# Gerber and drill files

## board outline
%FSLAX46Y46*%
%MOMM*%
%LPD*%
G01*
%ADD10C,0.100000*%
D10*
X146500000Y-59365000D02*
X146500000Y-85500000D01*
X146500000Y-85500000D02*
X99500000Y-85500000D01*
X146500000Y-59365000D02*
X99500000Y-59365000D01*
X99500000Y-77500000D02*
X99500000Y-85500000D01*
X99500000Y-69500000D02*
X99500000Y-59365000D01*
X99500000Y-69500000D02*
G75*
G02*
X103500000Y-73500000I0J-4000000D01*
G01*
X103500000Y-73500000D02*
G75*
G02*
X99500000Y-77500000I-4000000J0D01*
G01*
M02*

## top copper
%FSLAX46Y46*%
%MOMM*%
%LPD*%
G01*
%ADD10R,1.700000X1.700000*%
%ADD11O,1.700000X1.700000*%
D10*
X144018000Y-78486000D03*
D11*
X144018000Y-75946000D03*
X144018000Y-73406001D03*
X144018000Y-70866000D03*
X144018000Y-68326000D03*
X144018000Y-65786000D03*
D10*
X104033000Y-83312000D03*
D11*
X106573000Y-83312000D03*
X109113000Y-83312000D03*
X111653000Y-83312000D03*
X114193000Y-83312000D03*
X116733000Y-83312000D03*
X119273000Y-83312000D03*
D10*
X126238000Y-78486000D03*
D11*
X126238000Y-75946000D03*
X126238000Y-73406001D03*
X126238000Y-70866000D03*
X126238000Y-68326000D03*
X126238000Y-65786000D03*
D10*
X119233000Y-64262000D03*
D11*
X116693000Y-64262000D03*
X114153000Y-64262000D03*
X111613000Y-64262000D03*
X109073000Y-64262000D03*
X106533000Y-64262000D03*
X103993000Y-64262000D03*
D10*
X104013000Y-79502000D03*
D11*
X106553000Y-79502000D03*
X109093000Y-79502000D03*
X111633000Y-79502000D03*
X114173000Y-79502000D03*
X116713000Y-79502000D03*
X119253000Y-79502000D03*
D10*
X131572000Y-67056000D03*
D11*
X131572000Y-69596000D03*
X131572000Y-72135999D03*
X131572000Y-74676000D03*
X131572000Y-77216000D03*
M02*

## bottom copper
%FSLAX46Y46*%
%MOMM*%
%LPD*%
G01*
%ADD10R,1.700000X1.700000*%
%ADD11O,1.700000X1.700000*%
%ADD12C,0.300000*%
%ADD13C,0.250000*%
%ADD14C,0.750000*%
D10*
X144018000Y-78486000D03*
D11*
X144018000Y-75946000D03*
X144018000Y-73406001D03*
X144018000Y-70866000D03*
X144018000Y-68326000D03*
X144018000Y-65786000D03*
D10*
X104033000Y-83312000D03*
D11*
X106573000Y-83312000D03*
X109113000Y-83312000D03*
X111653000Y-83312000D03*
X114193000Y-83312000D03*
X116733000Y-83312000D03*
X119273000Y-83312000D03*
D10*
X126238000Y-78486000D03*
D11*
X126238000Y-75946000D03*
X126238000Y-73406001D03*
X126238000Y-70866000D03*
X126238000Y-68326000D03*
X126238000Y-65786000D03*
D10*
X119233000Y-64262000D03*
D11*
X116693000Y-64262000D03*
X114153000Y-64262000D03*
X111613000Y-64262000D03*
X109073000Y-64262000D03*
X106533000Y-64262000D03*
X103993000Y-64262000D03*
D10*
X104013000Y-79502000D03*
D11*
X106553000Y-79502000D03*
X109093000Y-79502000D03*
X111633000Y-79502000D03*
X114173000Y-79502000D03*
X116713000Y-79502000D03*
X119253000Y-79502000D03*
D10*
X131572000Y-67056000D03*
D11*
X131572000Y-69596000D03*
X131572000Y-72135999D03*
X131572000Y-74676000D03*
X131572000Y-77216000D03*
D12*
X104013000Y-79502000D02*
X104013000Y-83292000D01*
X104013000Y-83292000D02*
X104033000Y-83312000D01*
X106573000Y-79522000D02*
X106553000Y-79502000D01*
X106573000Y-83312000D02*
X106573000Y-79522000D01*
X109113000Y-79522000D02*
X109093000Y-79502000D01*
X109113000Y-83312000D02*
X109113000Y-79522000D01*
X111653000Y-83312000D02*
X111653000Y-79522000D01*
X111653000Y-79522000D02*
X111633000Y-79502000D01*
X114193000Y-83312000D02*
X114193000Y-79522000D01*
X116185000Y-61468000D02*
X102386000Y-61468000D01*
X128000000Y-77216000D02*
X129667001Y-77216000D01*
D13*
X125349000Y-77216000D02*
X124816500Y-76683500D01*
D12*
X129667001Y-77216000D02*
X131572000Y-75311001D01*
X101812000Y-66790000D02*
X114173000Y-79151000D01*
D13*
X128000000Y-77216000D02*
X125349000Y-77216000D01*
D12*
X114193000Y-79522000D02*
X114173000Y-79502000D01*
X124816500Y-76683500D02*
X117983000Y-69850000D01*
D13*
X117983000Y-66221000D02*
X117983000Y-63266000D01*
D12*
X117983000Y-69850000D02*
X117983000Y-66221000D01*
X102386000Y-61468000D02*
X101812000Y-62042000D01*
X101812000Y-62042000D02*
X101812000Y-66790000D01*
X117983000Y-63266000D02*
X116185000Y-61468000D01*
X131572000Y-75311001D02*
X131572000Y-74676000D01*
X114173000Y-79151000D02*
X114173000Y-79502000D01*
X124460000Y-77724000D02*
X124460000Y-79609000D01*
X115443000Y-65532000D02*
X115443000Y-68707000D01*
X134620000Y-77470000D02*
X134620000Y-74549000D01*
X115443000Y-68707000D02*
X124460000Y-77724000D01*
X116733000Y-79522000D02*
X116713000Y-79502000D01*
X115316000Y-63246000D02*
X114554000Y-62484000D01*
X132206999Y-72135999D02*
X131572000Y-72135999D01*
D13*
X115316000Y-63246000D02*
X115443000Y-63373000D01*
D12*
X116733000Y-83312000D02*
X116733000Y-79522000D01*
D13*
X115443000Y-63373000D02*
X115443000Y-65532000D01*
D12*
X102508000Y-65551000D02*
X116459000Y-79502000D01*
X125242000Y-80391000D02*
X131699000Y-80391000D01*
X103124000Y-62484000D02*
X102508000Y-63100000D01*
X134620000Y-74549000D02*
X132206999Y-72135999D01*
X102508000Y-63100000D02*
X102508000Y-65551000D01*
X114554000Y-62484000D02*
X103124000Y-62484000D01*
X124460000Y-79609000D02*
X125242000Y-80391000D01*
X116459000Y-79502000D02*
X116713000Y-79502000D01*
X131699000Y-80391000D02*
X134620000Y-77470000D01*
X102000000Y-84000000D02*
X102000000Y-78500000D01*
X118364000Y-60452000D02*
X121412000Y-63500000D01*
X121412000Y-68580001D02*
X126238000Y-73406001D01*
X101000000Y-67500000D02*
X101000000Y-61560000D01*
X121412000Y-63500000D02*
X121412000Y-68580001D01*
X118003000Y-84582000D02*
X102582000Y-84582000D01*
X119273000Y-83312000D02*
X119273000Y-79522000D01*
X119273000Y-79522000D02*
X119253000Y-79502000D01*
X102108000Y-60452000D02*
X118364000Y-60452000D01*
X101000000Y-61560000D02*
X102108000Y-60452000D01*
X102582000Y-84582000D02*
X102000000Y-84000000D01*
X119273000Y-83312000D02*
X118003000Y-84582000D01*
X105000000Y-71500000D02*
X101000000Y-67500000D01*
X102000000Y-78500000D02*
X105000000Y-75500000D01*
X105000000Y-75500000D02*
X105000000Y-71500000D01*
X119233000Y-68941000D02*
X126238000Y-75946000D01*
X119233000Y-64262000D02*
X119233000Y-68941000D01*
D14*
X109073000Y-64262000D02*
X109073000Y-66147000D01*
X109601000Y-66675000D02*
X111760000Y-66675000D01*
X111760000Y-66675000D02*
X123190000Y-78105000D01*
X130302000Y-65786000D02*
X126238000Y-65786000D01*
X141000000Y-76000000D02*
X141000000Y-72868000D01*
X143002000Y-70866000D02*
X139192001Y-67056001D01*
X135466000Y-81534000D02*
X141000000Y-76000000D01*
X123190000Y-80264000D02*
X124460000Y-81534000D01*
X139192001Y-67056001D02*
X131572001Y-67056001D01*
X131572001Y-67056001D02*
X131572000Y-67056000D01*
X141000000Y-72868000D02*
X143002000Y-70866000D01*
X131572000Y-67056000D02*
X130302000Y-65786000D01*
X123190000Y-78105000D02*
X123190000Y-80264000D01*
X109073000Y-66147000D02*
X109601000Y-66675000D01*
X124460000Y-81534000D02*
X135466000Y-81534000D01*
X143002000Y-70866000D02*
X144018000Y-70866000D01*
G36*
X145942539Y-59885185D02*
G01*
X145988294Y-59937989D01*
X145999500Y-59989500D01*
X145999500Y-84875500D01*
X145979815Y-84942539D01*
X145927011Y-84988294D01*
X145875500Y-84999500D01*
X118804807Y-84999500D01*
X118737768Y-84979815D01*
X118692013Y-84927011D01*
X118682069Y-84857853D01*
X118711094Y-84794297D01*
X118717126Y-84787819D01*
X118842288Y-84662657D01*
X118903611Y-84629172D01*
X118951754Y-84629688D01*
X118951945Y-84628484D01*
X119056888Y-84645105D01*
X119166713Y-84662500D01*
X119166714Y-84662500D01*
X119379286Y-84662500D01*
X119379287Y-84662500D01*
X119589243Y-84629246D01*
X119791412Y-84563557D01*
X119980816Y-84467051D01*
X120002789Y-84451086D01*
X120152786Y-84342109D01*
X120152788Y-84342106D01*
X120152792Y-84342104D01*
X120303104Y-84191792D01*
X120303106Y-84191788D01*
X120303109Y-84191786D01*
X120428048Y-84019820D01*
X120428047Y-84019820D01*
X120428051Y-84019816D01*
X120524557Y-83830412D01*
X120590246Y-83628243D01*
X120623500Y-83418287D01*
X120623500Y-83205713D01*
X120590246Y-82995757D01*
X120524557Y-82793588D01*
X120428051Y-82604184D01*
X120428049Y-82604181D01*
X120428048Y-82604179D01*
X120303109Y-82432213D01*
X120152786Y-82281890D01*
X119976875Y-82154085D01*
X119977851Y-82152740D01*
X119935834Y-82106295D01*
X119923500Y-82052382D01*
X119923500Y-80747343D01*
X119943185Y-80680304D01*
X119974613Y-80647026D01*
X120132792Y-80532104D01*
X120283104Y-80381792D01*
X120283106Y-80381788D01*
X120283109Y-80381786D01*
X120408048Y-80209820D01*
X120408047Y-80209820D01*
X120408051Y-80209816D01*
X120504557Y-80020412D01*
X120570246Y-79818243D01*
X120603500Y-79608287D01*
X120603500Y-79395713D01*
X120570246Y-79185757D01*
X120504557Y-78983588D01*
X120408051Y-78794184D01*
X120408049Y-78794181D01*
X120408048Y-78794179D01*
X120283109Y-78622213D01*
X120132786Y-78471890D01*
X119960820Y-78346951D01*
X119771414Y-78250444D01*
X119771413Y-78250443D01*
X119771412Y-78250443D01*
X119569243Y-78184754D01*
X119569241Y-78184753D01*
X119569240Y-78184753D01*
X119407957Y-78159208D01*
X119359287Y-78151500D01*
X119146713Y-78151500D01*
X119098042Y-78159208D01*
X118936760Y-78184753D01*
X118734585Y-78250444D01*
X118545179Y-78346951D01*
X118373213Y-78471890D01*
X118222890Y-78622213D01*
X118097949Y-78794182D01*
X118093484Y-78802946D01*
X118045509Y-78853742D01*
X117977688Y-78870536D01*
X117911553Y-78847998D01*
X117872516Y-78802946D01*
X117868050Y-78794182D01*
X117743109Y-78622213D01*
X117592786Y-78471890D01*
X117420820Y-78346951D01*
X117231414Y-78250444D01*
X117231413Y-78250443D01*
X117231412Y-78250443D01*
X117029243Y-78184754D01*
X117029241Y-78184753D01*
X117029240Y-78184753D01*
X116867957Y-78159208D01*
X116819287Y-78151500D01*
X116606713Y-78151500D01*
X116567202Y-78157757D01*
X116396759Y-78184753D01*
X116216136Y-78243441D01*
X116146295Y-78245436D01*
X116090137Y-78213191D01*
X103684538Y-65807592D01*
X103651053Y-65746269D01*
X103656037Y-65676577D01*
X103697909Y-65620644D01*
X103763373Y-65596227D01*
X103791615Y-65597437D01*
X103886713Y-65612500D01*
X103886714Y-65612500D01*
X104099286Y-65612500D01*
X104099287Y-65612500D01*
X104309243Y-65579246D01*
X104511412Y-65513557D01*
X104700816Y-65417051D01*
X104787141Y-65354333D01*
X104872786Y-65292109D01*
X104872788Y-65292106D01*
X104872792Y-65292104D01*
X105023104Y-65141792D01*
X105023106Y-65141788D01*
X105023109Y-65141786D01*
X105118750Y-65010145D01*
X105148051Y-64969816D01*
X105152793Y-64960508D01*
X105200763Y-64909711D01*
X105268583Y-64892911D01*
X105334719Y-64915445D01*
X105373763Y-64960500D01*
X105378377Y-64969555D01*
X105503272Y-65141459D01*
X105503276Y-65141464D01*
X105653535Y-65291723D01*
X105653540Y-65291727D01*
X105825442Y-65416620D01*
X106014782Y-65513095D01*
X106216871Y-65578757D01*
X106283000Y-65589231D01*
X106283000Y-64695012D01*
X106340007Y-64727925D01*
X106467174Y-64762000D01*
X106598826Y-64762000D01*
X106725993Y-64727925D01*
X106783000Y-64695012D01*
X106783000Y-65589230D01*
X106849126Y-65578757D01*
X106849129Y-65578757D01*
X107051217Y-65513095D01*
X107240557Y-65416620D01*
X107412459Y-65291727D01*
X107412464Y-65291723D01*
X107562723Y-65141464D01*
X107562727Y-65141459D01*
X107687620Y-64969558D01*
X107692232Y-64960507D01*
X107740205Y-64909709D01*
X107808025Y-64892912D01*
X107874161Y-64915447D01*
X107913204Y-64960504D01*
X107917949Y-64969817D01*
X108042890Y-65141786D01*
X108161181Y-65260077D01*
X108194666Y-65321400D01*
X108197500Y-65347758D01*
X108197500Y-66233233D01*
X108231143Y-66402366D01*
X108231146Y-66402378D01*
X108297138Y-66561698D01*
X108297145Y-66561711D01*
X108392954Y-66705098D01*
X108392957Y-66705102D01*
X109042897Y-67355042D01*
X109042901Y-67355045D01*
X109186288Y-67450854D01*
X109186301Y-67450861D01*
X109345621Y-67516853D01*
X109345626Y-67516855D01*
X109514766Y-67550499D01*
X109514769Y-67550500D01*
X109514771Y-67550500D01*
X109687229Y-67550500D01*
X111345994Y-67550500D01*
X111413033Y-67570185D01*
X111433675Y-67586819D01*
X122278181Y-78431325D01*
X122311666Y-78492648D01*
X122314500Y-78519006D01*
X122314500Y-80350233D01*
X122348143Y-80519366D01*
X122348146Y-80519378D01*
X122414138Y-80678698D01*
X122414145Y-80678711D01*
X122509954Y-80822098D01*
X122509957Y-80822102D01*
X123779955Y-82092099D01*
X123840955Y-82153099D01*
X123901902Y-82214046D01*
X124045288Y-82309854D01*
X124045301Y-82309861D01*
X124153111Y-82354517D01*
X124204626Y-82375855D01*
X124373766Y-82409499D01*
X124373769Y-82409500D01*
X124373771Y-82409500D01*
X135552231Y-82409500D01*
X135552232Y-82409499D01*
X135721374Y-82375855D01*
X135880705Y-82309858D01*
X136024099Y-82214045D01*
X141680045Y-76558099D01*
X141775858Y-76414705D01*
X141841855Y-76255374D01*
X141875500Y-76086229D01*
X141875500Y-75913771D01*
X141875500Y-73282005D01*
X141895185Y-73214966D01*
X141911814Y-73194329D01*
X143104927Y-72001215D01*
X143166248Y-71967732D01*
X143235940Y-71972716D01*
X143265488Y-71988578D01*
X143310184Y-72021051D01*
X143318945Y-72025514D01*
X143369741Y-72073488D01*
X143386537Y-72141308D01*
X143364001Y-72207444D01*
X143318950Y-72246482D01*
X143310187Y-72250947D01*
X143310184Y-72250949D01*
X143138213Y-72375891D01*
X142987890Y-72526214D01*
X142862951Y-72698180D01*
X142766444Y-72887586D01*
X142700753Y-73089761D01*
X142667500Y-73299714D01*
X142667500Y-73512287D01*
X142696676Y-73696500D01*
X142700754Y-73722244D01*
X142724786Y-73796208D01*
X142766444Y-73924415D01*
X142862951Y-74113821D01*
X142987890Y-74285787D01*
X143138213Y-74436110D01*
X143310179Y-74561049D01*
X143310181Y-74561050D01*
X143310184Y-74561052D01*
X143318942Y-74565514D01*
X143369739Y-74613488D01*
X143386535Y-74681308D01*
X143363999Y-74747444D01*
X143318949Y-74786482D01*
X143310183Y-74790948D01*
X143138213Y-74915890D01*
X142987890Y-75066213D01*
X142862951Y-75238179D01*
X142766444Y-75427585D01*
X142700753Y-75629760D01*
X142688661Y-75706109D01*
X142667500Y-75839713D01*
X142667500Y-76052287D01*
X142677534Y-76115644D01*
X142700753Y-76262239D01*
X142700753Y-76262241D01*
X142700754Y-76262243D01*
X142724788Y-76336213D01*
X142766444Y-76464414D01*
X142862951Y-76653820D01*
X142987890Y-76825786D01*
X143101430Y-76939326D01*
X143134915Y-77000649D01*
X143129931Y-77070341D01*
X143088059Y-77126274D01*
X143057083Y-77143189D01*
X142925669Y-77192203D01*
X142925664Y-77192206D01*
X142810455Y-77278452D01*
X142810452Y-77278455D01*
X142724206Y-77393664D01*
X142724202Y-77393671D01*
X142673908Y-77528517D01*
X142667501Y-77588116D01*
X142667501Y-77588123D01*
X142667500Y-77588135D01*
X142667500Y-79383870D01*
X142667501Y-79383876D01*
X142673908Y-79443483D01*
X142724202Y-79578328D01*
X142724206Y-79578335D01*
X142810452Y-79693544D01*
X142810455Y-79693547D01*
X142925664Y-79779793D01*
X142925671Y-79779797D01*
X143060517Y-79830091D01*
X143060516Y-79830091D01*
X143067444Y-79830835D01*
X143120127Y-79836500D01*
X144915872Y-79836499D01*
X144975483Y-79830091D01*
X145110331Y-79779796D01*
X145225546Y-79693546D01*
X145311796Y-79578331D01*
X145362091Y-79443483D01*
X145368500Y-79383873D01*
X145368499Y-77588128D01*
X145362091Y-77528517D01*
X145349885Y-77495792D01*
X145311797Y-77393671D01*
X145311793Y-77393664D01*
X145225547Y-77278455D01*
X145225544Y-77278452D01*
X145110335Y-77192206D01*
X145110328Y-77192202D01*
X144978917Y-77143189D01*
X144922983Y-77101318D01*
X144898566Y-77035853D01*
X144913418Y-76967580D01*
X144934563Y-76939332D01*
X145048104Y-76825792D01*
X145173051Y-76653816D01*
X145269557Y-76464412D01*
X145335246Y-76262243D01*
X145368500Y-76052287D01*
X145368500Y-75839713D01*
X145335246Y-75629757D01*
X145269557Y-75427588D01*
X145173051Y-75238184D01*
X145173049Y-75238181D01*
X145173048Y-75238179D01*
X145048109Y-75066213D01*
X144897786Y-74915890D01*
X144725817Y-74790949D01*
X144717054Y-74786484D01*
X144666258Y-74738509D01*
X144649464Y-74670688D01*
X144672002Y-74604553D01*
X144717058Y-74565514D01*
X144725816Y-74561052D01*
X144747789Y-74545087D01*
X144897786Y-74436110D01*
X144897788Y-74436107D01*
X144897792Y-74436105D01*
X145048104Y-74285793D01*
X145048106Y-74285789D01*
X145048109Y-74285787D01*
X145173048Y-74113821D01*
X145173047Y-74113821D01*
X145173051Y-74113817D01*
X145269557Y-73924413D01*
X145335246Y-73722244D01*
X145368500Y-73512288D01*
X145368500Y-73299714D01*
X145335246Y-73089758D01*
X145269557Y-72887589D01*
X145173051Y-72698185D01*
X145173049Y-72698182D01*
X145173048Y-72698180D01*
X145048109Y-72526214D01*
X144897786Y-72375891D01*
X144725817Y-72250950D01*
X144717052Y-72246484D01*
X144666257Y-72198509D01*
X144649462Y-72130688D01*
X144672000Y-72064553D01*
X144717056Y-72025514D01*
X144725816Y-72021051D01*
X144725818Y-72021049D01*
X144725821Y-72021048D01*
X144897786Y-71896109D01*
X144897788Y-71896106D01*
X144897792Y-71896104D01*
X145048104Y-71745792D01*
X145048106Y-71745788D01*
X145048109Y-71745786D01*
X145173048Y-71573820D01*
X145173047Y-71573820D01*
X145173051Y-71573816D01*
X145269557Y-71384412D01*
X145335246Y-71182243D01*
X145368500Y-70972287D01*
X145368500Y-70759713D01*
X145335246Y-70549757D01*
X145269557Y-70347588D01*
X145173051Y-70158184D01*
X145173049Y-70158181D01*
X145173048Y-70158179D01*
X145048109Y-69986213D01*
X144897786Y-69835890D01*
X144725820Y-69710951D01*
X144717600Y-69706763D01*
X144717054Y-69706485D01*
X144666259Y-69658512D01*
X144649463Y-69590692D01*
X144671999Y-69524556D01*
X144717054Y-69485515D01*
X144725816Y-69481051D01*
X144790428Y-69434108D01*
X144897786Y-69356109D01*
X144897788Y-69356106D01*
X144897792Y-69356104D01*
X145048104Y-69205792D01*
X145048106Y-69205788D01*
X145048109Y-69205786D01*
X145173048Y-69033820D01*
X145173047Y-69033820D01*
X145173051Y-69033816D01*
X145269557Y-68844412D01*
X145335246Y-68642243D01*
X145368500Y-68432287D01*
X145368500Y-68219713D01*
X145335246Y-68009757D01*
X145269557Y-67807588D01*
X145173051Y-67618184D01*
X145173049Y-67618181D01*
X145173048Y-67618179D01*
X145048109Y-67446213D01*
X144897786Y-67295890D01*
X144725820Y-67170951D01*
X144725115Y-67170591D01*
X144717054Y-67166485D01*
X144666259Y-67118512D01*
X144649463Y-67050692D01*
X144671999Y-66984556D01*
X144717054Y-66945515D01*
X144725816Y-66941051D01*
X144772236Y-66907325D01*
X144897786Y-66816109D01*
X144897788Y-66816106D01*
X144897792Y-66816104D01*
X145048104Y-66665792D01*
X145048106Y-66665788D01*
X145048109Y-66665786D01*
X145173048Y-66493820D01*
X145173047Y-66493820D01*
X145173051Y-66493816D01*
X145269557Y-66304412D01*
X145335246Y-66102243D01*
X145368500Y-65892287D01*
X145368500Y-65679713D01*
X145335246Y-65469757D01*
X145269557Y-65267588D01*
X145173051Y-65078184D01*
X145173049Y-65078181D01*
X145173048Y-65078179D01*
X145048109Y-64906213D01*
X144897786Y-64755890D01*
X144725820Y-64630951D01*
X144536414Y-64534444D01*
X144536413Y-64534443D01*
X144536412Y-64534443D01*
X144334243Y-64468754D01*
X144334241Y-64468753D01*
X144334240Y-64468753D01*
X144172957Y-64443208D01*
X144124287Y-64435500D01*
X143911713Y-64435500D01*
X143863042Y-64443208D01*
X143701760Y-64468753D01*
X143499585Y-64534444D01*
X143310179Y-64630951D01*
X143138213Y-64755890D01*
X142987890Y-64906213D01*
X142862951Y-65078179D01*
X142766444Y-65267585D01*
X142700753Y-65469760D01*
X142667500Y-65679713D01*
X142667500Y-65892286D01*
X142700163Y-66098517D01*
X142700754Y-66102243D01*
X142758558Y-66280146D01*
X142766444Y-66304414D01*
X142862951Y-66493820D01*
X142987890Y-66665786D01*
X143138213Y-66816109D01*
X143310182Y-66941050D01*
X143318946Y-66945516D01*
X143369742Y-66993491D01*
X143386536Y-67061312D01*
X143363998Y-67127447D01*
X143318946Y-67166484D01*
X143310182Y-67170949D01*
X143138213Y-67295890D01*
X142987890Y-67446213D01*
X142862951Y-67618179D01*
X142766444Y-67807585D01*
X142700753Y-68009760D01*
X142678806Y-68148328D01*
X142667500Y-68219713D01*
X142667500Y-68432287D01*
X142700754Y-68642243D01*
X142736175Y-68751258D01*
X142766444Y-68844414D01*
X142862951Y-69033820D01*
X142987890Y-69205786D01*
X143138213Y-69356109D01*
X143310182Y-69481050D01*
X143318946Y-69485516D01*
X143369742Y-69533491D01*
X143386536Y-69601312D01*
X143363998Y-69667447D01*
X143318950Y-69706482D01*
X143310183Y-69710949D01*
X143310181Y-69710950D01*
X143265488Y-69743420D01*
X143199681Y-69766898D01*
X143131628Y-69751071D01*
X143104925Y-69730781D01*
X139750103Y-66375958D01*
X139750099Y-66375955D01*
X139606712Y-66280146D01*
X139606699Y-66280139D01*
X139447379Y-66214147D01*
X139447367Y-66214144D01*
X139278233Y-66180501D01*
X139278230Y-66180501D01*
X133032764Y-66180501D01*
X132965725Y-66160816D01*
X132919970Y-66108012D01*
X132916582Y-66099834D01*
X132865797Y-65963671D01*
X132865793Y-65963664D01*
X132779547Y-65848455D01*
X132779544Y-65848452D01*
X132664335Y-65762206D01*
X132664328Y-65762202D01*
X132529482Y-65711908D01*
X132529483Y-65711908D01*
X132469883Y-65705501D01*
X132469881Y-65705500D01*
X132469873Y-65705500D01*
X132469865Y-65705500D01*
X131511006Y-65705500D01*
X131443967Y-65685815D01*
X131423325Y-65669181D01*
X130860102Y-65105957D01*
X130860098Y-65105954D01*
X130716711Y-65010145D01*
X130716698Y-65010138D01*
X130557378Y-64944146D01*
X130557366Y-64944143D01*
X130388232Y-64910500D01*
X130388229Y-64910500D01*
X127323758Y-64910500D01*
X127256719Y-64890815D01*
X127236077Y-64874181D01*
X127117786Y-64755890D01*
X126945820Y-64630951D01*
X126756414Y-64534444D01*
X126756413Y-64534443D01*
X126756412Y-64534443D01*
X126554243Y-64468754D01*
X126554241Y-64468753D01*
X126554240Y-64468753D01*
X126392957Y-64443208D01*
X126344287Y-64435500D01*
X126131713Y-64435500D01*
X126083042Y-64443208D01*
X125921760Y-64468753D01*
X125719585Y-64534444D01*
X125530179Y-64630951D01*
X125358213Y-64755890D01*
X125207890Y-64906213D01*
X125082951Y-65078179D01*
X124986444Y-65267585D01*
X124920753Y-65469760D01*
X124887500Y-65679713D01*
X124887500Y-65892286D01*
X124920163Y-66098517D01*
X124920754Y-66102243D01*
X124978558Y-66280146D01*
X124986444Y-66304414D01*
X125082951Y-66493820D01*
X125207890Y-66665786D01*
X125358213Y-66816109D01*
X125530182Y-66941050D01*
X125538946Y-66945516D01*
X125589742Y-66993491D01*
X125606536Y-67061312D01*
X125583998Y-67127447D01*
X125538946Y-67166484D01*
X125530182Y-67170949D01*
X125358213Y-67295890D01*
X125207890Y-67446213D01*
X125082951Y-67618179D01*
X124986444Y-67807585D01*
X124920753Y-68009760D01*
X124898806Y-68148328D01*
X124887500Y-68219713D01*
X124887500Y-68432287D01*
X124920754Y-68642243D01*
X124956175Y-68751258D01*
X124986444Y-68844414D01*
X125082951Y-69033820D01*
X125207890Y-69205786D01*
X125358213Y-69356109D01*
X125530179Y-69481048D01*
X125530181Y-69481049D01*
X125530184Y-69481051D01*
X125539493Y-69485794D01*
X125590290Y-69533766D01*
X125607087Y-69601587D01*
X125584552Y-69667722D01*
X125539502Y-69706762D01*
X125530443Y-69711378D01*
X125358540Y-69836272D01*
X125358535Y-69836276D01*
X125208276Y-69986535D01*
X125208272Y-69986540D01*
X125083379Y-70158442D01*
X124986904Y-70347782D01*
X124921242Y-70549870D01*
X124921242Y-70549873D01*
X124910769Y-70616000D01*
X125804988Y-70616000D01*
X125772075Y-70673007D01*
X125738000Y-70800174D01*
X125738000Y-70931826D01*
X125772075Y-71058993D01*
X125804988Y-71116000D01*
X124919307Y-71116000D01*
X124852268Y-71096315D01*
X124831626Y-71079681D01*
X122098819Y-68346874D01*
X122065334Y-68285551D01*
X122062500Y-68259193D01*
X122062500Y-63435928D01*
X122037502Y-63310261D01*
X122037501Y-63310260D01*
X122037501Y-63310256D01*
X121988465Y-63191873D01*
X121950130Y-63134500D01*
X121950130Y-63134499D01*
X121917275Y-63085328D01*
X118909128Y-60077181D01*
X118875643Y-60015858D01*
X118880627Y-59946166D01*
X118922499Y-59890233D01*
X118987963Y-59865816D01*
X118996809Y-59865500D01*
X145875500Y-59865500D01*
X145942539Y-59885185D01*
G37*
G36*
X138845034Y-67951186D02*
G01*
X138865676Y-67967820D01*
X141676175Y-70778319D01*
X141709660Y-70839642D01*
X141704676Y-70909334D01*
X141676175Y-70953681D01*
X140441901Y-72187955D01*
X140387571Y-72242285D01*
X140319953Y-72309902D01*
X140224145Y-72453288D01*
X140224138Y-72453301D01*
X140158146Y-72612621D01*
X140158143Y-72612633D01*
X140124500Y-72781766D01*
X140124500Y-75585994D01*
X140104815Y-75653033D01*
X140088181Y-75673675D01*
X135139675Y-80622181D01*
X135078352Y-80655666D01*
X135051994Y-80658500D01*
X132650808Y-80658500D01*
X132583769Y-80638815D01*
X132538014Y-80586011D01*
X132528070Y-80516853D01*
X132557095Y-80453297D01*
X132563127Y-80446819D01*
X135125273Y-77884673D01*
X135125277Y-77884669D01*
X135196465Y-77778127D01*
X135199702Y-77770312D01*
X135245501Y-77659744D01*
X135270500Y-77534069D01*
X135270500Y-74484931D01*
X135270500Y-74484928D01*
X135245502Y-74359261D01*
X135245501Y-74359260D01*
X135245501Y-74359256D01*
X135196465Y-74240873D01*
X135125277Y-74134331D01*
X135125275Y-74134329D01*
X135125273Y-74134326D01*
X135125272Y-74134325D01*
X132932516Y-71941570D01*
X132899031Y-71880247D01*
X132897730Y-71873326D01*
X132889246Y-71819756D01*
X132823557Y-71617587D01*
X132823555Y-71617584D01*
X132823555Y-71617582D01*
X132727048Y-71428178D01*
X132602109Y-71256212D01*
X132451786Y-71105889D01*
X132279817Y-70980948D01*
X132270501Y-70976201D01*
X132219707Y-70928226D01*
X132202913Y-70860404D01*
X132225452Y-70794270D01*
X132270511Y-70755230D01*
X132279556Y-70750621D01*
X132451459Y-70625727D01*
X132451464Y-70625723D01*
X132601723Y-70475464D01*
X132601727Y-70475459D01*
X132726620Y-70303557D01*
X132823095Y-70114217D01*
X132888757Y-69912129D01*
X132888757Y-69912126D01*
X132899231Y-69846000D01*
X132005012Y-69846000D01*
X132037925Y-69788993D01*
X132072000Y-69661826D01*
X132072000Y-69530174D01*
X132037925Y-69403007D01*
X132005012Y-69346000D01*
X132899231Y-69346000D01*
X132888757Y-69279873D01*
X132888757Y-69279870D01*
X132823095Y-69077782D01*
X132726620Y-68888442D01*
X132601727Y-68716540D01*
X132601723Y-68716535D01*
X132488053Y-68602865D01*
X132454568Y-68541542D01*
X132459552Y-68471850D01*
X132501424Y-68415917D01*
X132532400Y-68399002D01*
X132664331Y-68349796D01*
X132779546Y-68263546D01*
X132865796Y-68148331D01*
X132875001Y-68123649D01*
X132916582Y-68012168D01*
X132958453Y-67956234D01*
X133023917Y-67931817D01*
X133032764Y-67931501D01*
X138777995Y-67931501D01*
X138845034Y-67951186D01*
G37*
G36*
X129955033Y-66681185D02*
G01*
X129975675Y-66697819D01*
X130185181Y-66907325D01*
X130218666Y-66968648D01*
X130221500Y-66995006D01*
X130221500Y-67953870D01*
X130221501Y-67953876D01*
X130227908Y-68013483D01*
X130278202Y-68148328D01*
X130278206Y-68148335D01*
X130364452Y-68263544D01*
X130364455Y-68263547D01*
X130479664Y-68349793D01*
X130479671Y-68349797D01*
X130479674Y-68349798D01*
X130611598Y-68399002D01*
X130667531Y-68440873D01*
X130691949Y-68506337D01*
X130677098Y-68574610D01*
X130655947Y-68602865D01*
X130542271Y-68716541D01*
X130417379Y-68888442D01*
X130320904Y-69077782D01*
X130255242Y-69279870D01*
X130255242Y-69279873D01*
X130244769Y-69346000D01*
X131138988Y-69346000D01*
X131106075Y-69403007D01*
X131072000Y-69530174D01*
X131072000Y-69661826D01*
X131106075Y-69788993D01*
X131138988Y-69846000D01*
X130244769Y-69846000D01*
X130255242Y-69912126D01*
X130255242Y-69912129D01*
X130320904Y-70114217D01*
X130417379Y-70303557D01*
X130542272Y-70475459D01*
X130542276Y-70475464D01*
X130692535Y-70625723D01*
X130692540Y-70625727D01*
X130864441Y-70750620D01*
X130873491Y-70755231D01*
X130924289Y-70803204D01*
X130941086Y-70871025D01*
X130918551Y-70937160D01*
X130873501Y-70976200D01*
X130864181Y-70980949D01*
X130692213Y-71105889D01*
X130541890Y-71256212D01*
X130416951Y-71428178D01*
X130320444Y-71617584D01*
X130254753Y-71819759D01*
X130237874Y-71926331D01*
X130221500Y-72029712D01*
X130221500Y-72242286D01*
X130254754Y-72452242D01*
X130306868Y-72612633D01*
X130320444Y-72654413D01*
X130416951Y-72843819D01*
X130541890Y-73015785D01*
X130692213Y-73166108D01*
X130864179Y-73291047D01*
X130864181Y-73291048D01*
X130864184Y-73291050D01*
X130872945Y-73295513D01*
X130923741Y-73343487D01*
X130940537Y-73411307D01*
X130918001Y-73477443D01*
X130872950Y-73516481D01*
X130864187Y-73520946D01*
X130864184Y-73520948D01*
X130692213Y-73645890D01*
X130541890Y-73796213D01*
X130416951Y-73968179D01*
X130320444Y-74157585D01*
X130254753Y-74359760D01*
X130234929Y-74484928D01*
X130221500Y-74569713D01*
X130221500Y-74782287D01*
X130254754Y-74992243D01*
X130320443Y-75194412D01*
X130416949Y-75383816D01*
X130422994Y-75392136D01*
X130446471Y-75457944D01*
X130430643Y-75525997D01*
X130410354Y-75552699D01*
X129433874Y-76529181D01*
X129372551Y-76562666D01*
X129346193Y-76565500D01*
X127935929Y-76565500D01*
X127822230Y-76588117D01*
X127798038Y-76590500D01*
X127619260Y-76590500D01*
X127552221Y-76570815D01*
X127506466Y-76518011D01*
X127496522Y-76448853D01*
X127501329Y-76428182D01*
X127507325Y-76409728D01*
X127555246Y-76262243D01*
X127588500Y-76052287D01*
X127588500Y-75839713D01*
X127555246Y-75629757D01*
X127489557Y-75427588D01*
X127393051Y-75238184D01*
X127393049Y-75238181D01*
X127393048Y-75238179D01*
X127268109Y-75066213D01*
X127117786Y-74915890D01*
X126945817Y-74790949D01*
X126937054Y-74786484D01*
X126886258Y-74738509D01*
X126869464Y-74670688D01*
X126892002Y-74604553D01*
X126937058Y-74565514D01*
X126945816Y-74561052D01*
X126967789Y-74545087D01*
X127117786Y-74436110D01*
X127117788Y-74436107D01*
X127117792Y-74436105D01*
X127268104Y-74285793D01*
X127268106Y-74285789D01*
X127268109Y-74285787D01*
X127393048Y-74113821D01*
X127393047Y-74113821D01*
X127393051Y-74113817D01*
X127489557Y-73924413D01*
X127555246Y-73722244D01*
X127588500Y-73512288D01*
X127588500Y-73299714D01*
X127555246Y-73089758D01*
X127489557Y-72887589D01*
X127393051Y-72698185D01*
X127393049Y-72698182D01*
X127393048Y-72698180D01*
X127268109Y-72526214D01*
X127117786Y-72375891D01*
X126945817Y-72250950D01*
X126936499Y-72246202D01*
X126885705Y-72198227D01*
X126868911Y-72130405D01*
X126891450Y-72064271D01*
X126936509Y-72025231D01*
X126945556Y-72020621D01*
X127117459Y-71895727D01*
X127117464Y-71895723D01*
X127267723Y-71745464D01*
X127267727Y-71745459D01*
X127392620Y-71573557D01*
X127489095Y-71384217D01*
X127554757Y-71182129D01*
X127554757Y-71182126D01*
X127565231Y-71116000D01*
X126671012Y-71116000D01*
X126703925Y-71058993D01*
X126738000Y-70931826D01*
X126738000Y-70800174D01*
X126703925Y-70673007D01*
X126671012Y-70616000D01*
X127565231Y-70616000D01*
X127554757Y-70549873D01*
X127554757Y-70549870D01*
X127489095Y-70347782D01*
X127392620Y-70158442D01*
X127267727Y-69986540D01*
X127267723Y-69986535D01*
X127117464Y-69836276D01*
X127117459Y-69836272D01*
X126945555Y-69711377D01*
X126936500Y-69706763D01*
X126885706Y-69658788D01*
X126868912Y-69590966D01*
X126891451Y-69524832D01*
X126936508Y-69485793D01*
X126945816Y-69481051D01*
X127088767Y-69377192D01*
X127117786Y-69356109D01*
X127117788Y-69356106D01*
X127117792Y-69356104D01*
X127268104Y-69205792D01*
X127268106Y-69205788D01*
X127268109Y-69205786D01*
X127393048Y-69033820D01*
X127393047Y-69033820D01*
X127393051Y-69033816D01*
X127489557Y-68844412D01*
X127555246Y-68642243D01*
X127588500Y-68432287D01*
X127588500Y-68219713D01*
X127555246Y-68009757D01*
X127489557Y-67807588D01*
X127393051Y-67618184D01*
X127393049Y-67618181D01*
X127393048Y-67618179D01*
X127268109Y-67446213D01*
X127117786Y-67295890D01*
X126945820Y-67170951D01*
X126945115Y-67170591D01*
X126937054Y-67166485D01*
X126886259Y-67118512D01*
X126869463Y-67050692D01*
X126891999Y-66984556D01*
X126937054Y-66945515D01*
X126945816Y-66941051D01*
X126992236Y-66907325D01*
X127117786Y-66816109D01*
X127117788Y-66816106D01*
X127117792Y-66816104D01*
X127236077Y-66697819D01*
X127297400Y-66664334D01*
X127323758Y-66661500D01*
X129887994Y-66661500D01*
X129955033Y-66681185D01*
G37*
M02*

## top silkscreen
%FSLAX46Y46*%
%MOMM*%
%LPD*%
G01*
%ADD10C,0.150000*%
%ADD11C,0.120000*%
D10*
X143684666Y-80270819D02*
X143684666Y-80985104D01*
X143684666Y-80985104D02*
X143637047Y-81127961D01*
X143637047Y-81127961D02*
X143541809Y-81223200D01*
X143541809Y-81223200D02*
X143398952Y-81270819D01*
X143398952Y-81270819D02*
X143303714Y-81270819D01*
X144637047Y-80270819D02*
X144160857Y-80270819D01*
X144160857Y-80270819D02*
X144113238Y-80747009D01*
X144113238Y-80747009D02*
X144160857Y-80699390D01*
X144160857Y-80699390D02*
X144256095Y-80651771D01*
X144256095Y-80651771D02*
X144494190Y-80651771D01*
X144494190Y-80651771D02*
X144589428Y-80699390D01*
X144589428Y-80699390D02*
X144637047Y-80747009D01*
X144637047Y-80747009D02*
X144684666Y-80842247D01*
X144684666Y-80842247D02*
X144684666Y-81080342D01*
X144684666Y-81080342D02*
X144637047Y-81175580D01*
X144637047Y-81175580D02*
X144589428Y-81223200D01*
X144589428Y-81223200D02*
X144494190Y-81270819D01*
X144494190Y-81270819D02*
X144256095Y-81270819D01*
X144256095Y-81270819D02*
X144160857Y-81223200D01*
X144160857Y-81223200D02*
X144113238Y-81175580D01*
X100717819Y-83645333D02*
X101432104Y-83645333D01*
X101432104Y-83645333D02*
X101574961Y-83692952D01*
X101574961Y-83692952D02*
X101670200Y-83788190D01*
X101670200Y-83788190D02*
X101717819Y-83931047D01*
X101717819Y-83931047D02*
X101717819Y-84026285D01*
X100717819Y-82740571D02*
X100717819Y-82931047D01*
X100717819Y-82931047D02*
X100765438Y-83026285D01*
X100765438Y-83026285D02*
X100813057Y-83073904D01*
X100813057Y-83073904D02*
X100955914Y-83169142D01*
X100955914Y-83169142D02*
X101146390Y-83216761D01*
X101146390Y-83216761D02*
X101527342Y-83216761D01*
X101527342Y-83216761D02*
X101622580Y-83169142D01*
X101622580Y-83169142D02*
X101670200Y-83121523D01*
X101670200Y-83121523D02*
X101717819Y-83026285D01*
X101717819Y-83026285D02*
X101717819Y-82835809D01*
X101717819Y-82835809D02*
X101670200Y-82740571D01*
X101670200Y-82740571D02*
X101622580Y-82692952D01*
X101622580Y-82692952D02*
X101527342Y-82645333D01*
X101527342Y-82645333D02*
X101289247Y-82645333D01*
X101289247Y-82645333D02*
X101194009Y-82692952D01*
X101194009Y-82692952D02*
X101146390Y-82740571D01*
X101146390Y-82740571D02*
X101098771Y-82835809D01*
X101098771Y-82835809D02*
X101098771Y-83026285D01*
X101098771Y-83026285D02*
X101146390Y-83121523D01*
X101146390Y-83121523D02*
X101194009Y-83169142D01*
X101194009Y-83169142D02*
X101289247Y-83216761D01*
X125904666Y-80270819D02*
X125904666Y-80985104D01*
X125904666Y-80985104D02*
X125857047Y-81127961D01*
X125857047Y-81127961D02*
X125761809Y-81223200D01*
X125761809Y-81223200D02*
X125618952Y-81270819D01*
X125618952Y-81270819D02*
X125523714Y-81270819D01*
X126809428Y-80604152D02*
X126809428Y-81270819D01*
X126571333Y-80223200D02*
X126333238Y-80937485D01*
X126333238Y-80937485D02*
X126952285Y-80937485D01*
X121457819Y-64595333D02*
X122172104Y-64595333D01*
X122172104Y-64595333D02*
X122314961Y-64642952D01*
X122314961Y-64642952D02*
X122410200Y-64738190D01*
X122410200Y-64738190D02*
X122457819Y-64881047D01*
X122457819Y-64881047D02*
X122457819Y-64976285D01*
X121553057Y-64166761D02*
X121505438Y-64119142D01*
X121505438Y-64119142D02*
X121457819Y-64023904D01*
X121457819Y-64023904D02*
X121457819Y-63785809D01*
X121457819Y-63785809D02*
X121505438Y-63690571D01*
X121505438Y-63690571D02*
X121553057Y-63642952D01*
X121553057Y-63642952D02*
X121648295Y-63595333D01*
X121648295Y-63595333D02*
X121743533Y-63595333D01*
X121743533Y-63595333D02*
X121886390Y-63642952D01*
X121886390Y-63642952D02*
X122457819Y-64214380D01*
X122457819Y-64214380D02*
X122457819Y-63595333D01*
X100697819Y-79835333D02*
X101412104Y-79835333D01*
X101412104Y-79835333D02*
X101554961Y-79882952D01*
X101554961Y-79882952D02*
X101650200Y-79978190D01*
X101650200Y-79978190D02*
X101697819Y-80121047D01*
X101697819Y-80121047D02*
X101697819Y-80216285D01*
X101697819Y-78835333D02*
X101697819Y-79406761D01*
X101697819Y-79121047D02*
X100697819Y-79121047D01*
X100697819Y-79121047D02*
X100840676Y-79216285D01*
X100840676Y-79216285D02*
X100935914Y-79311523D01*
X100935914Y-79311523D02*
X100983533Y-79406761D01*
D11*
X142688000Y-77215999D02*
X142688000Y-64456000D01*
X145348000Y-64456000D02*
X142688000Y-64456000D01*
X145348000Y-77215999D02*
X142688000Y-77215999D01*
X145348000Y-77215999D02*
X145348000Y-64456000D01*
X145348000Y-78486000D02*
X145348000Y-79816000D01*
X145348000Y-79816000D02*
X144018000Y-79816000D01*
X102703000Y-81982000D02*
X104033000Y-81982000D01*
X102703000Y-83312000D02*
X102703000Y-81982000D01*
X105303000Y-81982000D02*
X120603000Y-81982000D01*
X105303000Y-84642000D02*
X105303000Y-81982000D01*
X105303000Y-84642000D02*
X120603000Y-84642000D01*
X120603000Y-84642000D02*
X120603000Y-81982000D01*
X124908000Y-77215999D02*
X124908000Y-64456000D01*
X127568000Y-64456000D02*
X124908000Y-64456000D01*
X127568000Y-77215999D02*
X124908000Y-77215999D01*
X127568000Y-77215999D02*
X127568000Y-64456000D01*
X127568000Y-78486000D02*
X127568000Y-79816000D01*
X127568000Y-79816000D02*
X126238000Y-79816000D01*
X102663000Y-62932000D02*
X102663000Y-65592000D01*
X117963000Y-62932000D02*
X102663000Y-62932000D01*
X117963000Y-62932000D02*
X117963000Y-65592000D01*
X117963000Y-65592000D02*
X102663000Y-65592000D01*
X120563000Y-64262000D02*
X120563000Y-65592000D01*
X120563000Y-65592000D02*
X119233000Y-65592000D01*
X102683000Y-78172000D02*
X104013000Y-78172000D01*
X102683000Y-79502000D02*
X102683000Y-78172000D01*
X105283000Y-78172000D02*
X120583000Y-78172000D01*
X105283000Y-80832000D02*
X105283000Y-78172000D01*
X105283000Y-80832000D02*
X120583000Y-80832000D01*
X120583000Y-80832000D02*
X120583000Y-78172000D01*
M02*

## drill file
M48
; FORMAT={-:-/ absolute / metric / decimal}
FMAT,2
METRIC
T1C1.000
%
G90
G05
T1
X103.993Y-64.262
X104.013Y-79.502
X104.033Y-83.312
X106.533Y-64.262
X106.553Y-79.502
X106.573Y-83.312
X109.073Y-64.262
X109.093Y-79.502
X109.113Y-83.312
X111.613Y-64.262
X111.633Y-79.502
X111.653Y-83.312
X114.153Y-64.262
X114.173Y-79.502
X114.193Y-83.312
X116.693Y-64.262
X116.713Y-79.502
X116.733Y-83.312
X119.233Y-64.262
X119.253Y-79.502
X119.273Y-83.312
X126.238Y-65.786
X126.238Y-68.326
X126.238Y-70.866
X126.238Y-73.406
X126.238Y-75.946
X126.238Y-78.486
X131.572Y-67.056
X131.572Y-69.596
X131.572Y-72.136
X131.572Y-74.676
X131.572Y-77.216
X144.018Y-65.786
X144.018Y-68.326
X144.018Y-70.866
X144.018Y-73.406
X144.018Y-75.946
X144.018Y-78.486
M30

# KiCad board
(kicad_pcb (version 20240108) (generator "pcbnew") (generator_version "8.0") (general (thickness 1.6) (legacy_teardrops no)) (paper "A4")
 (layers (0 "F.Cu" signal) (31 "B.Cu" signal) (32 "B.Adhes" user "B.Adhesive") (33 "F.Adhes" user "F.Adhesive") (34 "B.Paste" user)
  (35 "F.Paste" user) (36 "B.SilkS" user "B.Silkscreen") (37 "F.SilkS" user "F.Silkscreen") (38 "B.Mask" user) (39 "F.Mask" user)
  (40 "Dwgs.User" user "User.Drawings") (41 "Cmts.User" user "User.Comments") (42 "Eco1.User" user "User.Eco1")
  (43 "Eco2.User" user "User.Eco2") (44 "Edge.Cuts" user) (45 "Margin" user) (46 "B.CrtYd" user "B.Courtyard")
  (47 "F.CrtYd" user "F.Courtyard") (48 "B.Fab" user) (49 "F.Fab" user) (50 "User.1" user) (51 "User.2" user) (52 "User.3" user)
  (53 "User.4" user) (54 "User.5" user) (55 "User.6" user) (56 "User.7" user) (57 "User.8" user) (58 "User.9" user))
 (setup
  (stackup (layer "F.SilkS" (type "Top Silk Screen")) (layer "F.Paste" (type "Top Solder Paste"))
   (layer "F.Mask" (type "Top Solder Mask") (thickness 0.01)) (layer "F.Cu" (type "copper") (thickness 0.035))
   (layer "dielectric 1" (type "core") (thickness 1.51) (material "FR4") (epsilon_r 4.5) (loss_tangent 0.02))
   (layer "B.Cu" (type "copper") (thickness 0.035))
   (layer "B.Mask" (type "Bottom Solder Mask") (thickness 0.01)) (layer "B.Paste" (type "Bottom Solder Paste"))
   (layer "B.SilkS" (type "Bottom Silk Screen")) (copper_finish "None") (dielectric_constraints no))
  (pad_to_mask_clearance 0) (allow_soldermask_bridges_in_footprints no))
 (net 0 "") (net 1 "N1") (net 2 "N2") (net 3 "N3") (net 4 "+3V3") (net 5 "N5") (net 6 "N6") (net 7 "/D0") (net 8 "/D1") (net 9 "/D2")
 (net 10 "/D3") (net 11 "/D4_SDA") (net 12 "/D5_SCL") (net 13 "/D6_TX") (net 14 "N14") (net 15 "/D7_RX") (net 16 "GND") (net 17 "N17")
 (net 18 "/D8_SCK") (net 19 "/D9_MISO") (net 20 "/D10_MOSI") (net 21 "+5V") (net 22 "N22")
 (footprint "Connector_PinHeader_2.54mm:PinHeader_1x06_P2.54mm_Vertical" (layer "F.Cu") (at 144.018 78.486 180)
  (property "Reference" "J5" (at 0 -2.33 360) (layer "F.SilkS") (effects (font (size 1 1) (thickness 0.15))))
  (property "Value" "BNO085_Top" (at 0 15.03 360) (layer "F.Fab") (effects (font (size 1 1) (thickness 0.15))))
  (fp_line (start 1.33 1.270001) (end 1.33 14.03) (stroke (width 0.12) (type solid)) (layer "F.SilkS"))
  (fp_line (start -1.33 14.03) (end 1.33 14.03) (stroke (width 0.12) (type solid)) (layer "F.SilkS"))
  (fp_line (start -1.33 1.270001) (end 1.33 1.270001) (stroke (width 0.12) (type solid)) (layer "F.SilkS"))
  (fp_line (start -1.33 1.270001) (end -1.33 14.03) (stroke (width 0.12) (type solid)) (layer "F.SilkS"))
  (fp_line (start -1.33 0) (end -1.33 -1.33) (stroke (width 0.12) (type solid)) (layer "F.SilkS"))
  (fp_line (start -1.33 -1.33) (end 0 -1.33) (stroke (width 0.12) (type solid)) (layer "F.SilkS"))
  (pad "1" thru_hole rect (at 0 0 180) (size 1.7 1.7) (drill 1) (layers "*.Cu" "*.Mask") (remove_unused_layers no) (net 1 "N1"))
  (pad "2" thru_hole oval (at 0 2.54 180) (size 1.7 1.7) (drill 1) (layers "*.Cu" "*.Mask") (remove_unused_layers no) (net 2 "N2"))
  (pad "3" thru_hole oval (at 0 5.079999 180) (size 1.7 1.7) (drill 1) (layers "*.Cu" "*.Mask") (remove_unused_layers no) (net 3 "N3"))
  (pad "4" thru_hole oval (at 0 7.62 180) (size 1.7 1.7) (drill 1) (layers "*.Cu" "*.Mask") (remove_unused_layers no) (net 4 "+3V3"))
  (pad "5" thru_hole oval (at 0 10.16 180) (size 1.7 1.7) (drill 1) (layers "*.Cu" "*.Mask") (remove_unused_layers no) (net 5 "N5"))
  (pad "6" thru_hole oval (at 0 12.7 180) (size 1.7 1.7) (drill 1) (layers "*.Cu" "*.Mask") (remove_unused_layers no) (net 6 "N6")))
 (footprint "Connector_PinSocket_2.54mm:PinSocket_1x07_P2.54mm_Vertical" (layer "F.Cu") (at 104.033 83.312 90)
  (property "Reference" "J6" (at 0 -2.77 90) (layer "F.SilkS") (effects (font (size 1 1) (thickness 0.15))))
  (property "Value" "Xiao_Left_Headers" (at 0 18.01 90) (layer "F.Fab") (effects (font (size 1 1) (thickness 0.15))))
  (fp_line (start 1.33 -1.33) (end 1.33 0) (stroke (width 0.12) (type solid)) (layer "F.SilkS"))
  (fp_line (start 0 -1.33) (end 1.33 -1.33) (stroke (width 0.12) (type solid)) (layer "F.SilkS"))
  (fp_line (start 1.33 1.27) (end 1.33 16.57) (stroke (width 0.12) (type solid)) (layer "F.SilkS"))
  (fp_line (start -1.33 1.27) (end 1.33 1.27) (stroke (width 0.12) (type solid)) (layer "F.SilkS"))
  (fp_line (start -1.33 1.27) (end -1.33 16.57) (stroke (width 0.12) (type solid)) (layer "F.SilkS"))
  (fp_line (start -1.33 16.57) (end 1.33 16.57) (stroke (width 0.12) (type solid)) (layer "F.SilkS"))
  (pad "1" thru_hole rect (at 0 0 90) (size 1.7 1.7) (drill 1) (layers "*.Cu" "*.Mask") (remove_unused_layers no) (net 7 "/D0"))
  (pad "2" thru_hole oval (at 0 2.54 90) (size 1.7 1.7) (drill 1) (layers "*.Cu" "*.Mask") (remove_unused_layers no) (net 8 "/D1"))
  (pad "3" thru_hole oval (at 0 5.08 90) (size 1.7 1.7) (drill 1) (layers "*.Cu" "*.Mask") (remove_unused_layers no) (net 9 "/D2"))
  (pad "4" thru_hole oval (at 0 7.62 90) (size 1.7 1.7) (drill 1) (layers "*.Cu" "*.Mask") (remove_unused_layers no) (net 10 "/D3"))
  (pad "5" thru_hole oval (at 0 10.16 90) (size 1.7 1.7) (drill 1) (layers "*.Cu" "*.Mask") (remove_unused_layers no) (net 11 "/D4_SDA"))
  (pad "6" thru_hole oval (at 0 12.7 90) (size 1.7 1.7) (drill 1) (layers "*.Cu" "*.Mask") (remove_unused_layers no) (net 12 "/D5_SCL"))
  (pad "7" thru_hole oval (at 0 15.24 90) (size 1.7 1.7) (drill 1) (layers "*.Cu" "*.Mask") (remove_unused_layers no) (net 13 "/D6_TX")))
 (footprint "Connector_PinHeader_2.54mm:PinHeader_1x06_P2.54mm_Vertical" (layer "F.Cu") (at 126.238 78.486 180)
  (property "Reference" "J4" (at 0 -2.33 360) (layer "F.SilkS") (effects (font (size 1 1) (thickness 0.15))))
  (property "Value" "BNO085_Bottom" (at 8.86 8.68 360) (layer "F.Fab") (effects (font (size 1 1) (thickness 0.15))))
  (fp_line (start 1.33 1.270001) (end 1.33 14.03) (stroke (width 0.12) (type solid)) (layer "F.SilkS"))
  (fp_line (start -1.33 14.03) (end 1.33 14.03) (stroke (width 0.12) (type solid)) (layer "F.SilkS"))
  (fp_line (start -1.33 1.270001) (end 1.33 1.270001) (stroke (width 0.12) (type solid)) (layer "F.SilkS"))
  (fp_line (start -1.33 1.270001) (end -1.33 14.03) (stroke (width 0.12) (type solid)) (layer "F.SilkS"))
  (fp_line (start -1.33 0) (end -1.33 -1.33) (stroke (width 0.12) (type solid)) (layer "F.SilkS"))
  (fp_line (start -1.33 -1.33) (end 0 -1.33) (stroke (width 0.12) (type solid)) (layer "F.SilkS"))
  (pad "1" thru_hole rect (at 0 0 180) (size 1.7 1.7) (drill 1) (layers "*.Cu" "*.Mask") (remove_unused_layers no) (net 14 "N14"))
  (pad "2" thru_hole oval (at 0 2.54 180) (size 1.7 1.7) (drill 1) (layers "*.Cu" "*.Mask") (remove_unused_layers no) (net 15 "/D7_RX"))
  (pad "3" thru_hole oval (at 0 5.079999 180) (size 1.7 1.7) (drill 1) (layers "*.Cu" "*.Mask") (remove_unused_layers no) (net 13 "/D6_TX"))
  (pad "4" thru_hole oval (at 0 7.62 180) (size 1.7 1.7) (drill 1) (layers "*.Cu" "*.Mask") (remove_unused_layers no) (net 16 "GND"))
  (pad "5" thru_hole oval (at 0 10.16 180) (size 1.7 1.7) (drill 1) (layers "*.Cu" "*.Mask") (remove_unused_layers no) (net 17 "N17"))
  (pad "6" thru_hole oval (at 0 12.7 180) (size 1.7 1.7) (drill 1) (layers "*.Cu" "*.Mask") (remove_unused_layers no) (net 4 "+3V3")))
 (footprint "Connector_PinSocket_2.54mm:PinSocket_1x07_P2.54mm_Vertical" (layer "F.Cu") (at 119.233 64.262 -90)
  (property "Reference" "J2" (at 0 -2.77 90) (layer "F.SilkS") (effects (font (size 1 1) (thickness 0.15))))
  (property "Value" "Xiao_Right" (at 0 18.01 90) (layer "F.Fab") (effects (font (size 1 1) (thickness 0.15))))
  (fp_line (start -1.33 16.57) (end 1.33 16.57) (stroke (width 0.12) (type solid)) (layer "F.SilkS"))
  (fp_line (start -1.33 1.27) (end -1.33 16.57) (stroke (width 0.12) (type solid)) (layer "F.SilkS"))
  (fp_line (start -1.33 1.27) (end 1.33 1.27) (stroke (width 0.12) (type solid)) (layer "F.SilkS"))
  (fp_line (start 1.33 1.27) (end 1.33 16.57) (stroke (width 0.12) (type solid)) (layer "F.SilkS"))
  (fp_line (start 0 -1.33) (end 1.33 -1.33) (stroke (width 0.12) (type solid)) (layer "F.SilkS"))
  (fp_line (start 1.33 -1.33) (end 1.33 0) (stroke (width 0.12) (type solid)) (layer "F.SilkS"))
  (pad "1" thru_hole rect (at 0 0 270) (size 1.7 1.7) (drill 1) (layers "*.Cu" "*.Mask") (remove_unused_layers no) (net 15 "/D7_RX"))
  (pad "2" thru_hole oval (at 0 2.54 270) (size 1.7 1.7) (drill 1) (layers "*.Cu" "*.Mask") (remove_unused_layers no) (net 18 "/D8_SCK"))
  (pad "3" thru_hole oval (at 0 5.08 270) (size 1.7 1.7) (drill 1) (layers "*.Cu" "*.Mask") (remove_unused_layers no) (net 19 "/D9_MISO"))
  (pad "4" thru_hole oval (at 0 7.62 270) (size 1.7 1.7) (drill 1) (layers "*.Cu" "*.Mask") (remove_unused_layers no) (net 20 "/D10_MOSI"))
  (pad "5" thru_hole oval (at 0 10.16 270) (size 1.7 1.7) (drill 1) (layers "*.Cu" "*.Mask") (remove_unused_layers no) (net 4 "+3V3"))
  (pad "6" thru_hole oval (at 0 12.7 270) (size 1.7 1.7) (drill 1) (layers "*.Cu" "*.Mask") (remove_unused_layers no) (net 16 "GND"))
  (pad "7" thru_hole oval (at 0 15.24 270) (size 1.7 1.7) (drill 1) (layers "*.Cu" "*.Mask") (remove_unused_layers no) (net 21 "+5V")))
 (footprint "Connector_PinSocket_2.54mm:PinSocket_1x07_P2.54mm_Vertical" (layer "F.Cu") (at 104.013 79.502 90)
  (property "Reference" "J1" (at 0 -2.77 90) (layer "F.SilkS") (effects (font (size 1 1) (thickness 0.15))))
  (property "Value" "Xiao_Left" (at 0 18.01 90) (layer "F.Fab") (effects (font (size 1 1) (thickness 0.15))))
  (fp_line (start 1.33 -1.33) (end 1.33 0) (stroke (width 0.12) (type solid)) (layer "F.SilkS"))
  (fp_line (start 0 -1.33) (end 1.33 -1.33) (stroke (width 0.12) (type solid)) (layer "F.SilkS"))
  (fp_line (start 1.33 1.27) (end 1.33 16.57) (stroke (width 0.12) (type solid)) (layer "F.SilkS"))
  (fp_line (start -1.33 1.27) (end 1.33 1.27) (stroke (width 0.12) (type solid)) (layer "F.SilkS"))
  (fp_line (start -1.33 1.27) (end -1.33 16.57) (stroke (width 0.12) (type solid)) (layer "F.SilkS"))
  (fp_line (start -1.33 16.57) (end 1.33 16.57) (stroke (width 0.12) (type solid)) (layer "F.SilkS"))
  (pad "1" thru_hole rect (at 0 0 90) (size 1.7 1.7) (drill 1) (layers "*.Cu" "*.Mask") (remove_unused_layers no) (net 7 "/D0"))
  (pad "2" thru_hole oval (at 0 2.54 90) (size 1.7 1.7) (drill 1) (layers "*.Cu" "*.Mask") (remove_unused_layers no) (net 8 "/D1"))
  (pad "3" thru_hole oval (at 0 5.08 90) (size 1.7 1.7) (drill 1) (layers "*.Cu" "*.Mask") (remove_unused_layers no) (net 9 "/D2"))
  (pad "4" thru_hole oval (at 0 7.62 90) (size 1.7 1.7) (drill 1) (layers "*.Cu" "*.Mask") (remove_unused_layers no) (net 10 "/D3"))
  (pad "5" thru_hole oval (at 0 10.16 90) (size 1.7 1.7) (drill 1) (layers "*.Cu" "*.Mask") (remove_unused_layers no) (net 11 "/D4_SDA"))
  (pad "6" thru_hole oval (at 0 12.7 90) (size 1.7 1.7) (drill 1) (layers "*.Cu" "*.Mask") (remove_unused_layers no) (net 12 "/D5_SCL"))
  (pad "7" thru_hole oval (at 0 15.24 90) (size 1.7 1.7) (drill 1) (layers "*.Cu" "*.Mask") (remove_unused_layers no) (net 13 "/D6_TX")))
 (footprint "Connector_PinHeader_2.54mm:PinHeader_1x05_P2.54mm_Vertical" (layer "B.Cu") (at 131.572 67.056 180)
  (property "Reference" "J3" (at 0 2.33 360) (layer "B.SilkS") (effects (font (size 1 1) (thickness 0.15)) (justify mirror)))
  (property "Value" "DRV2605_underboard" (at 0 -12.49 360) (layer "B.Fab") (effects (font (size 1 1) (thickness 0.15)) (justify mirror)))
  (pad "1" thru_hole rect (at 0 0 180) (size 1.7 1.7) (drill 1) (layers "*.Cu" "*.Mask") (remove_unused_layers no) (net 4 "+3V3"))
  (pad "2" thru_hole oval (at 0 -2.54 180) (size 1.7 1.7) (drill 1) (layers "*.Cu" "*.Mask") (remove_unused_layers no) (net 16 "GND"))
  (pad "3" thru_hole oval (at 0 -5.079999 180) (size 1.7 1.7) (drill 1) (layers "*.Cu" "*.Mask") (remove_unused_layers no)
   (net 12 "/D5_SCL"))
  (pad "4" thru_hole oval (at 0 -7.62 180) (size 1.7 1.7) (drill 1) (layers "*.Cu" "*.Mask") (remove_unused_layers no) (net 11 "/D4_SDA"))
  (pad "5" thru_hole oval (at 0 -10.16 180) (size 1.7 1.7) (drill 1) (layers "*.Cu" "*.Mask") (remove_unused_layers no) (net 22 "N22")))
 (gr_line (start 146.5 59.365) (end 146.5 85.5) (stroke (width 0.1) (type default)) (layer "Edge.Cuts"))
 (gr_line (start 146.5 85.5) (end 99.5 85.5) (stroke (width 0.1) (type default)) (layer "Edge.Cuts"))
 (gr_line (start 146.5 59.365) (end 99.5 59.365) (stroke (width 0.1) (type default)) (layer "Edge.Cuts"))
 (gr_line (start 99.5 77.5) (end 99.5 85.5) (stroke (width 0.1) (type default)) (layer "Edge.Cuts"))
 (gr_line (start 99.5 69.5) (end 99.5 59.365) (stroke (width 0.1) (type default)) (layer "Edge.Cuts"))
 (gr_arc (start 99.5 69.5) (mid 102.328427 70.671573) (end 103.5 73.5) (stroke (width 0.1) (type default)) (layer "Edge.Cuts"))
 (gr_arc (start 103.5 73.5) (mid 102.328427 76.328427) (end 99.5 77.5) (stroke (width 0.1) (type default)) (layer "Edge.Cuts"))
 (segment (start 104.013 79.502) (end 104.013 83.292) (width 0.3) (layer "B.Cu") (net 7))
 (segment (start 104.013 83.292) (end 104.033 83.312) (width 0.3) (layer "B.Cu") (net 7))
 (segment (start 106.573 79.522) (end 106.553 79.502) (width 0.3) (layer "B.Cu") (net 8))
 (segment (start 106.573 83.312) (end 106.573 79.522) (width 0.3) (layer "B.Cu") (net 8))
 (segment (start 109.113 79.522) (end 109.093 79.502) (width 0.3) (layer "B.Cu") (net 9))
 (segment (start 109.113 83.312) (end 109.113 79.522) (width 0.3) (layer "B.Cu") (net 9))
 (segment (start 111.653 83.312) (end 111.653 79.522) (width 0.3) (layer "B.Cu") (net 10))
 (segment (start 111.653 79.522) (end 111.633 79.502) (width 0.3) (layer "B.Cu") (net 10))
 (segment (start 114.193 83.312) (end 114.193 79.522) (width 0.3) (layer "B.Cu") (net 11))
 (segment (start 116.185 61.468) (end 102.386 61.468) (width 0.3) (layer "B.Cu") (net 11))
 (segment (start 128 77.216) (end 129.667001 77.216) (width 0.3) (layer "B.Cu") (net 11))
 (segment (start 125.349 77.216) (end 124.8165 76.6835) (width 0.25) (layer "B.Cu") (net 11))
 (segment (start 129.667001 77.216) (end 131.572 75.311001) (width 0.3) (layer "B.Cu") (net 11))
 (segment (start 101.812 66.79) (end 114.173 79.151) (width 0.3) (layer "B.Cu") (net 11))
 (segment (start 128 77.216) (end 125.349 77.216) (width 0.25) (layer "B.Cu") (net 11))
 (segment (start 114.193 79.522) (end 114.173 79.502) (width 0.3) (layer "B.Cu") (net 11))
 (segment (start 124.8165 76.6835) (end 117.983 69.85) (width 0.3) (layer "B.Cu") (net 11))
 (segment (start 117.983 66.221) (end 117.983 63.266) (width 0.25) (layer "B.Cu") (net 11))
 (segment (start 117.983 69.85) (end 117.983 66.221) (width 0.3) (layer "B.Cu") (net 11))
 (segment (start 102.386 61.468) (end 101.812 62.042) (width 0.3) (layer "B.Cu") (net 11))
 (segment (start 101.812 62.042) (end 101.812 66.79) (width 0.3) (layer "B.Cu") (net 11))
 (segment (start 117.983 63.266) (end 116.185 61.468) (width 0.3) (layer "B.Cu") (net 11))
 (segment (start 131.572 75.311001) (end 131.572 74.676) (width 0.3) (layer "B.Cu") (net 11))
 (segment (start 114.173 79.151) (end 114.173 79.502) (width 0.3) (layer "B.Cu") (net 11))
 (segment (start 124.46 77.724) (end 124.46 79.609) (width 0.3) (layer "B.Cu") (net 12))
 (segment (start 115.443 65.532) (end 115.443 68.707) (width 0.3) (layer "B.Cu") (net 12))
 (segment (start 134.62 77.47) (end 134.62 74.549) (width 0.3) (layer "B.Cu") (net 12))
 (segment (start 115.443 68.707) (end 124.46 77.724) (width 0.3) (layer "B.Cu") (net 12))
 (segment (start 116.733 79.522) (end 116.713 79.502) (width 0.3) (layer "B.Cu") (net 12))
 (segment (start 115.316 63.246) (end 114.554 62.484) (width 0.3) (layer "B.Cu") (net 12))
 (segment (start 132.206999 72.135999) (end 131.572 72.135999) (width 0.3) (layer "B.Cu") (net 12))
 (segment (start 115.316 63.246) (end 115.443 63.373) (width 0.25) (layer "B.Cu") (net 12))
 (segment (start 116.733 83.312) (end 116.733 79.522) (width 0.3) (layer "B.Cu") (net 12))
 (segment (start 115.443 63.373) (end 115.443 65.532) (width 0.25) (layer "B.Cu") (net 12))
 (segment (start 102.508 65.551) (end 116.459 79.502) (width 0.3) (layer "B.Cu") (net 12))
 (segment (start 125.242 80.391) (end 131.699 80.391) (width 0.3) (layer "B.Cu") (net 12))
 (segment (start 103.124 62.484) (end 102.508 63.1) (width 0.3) (layer "B.Cu") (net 12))
 (segment (start 134.62 74.549) (end 132.206999 72.135999) (width 0.3) (layer "B.Cu") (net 12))
 (segment (start 102.508 63.1) (end 102.508 65.551) (width 0.3) (layer "B.Cu") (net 12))
 (segment (start 114.554 62.484) (end 103.124 62.484) (width 0.3) (layer "B.Cu") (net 12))
 (segment (start 124.46 79.609) (end 125.242 80.391) (width 0.3) (layer "B.Cu") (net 12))
 (segment (start 116.459 79.502) (end 116.713 79.502) (width 0.3) (layer "B.Cu") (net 12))
 (segment (start 131.699 80.391) (end 134.62 77.47) (width 0.3) (layer "B.Cu") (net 12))
 (segment (start 102 84) (end 102 78.5) (width 0.3) (layer "B.Cu") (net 13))
 (segment (start 118.364 60.452) (end 121.412 63.5) (width 0.3) (layer "B.Cu") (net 13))
 (segment (start 121.412 68.580001) (end 126.238 73.406001) (width 0.3) (layer "B.Cu") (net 13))
 (segment (start 101 67.5) (end 101 61.56) (width 0.3) (layer "B.Cu") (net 13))
 (segment (start 121.412 63.5) (end 121.412 68.580001) (width 0.3) (layer "B.Cu") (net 13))
 (segment (start 118.003 84.582) (end 102.582 84.582) (width 0.3) (layer "B.Cu") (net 13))
 (segment (start 119.273 83.312) (end 119.273 79.522) (width 0.3) (layer "B.Cu") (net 13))
 (segment (start 119.273 79.522) (end 119.253 79.502) (width 0.3) (layer "B.Cu") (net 13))
 (segment (start 102.108 60.452) (end 118.364 60.452) (width 0.3) (layer "B.Cu") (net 13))
 (segment (start 101 61.56) (end 102.108 60.452) (width 0.3) (layer "B.Cu") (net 13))
 (segment (start 102.582 84.582) (end 102 84) (width 0.3) (layer "B.Cu") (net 13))
 (segment (start 119.273 83.312) (end 118.003 84.582) (width 0.3) (layer "B.Cu") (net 13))
 (segment (start 105 71.5) (end 101 67.5) (width 0.3) (layer "B.Cu") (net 13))
 (segment (start 102 78.5) (end 105 75.5) (width 0.3) (layer "B.Cu") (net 13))
 (segment (start 105 75.5) (end 105 71.5) (width 0.3) (layer "B.Cu") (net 13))
 (segment (start 119.233 68.941) (end 126.238 75.946) (width 0.3) (layer "B.Cu") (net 15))
 (segment (start 119.233 64.262) (end 119.233 68.941) (width 0.3) (layer "B.Cu") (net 15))
 (segment (start 109.073 64.262) (end 109.073 66.147) (width 0.75) (layer "B.Cu") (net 4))
 (segment (start 109.601 66.675) (end 111.76 66.675) (width 0.75) (layer "B.Cu") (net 4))
 (segment (start 111.76 66.675) (end 123.19 78.105) (width 0.75) (layer "B.Cu") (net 4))
 (segment (start 130.302 65.786) (end 126.238 65.786) (width 0.75) (layer "B.Cu") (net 4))
 (segment (start 141 76) (end 141 72.868) (width 0.75) (layer "B.Cu") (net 4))
 (segment (start 143.002 70.866) (end 139.192001 67.056001) (width 0.75) (layer "B.Cu") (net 4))
 (segment (start 135.466 81.534) (end 141 76) (width 0.75) (layer "B.Cu") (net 4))
 (segment (start 123.19 80.264) (end 124.46 81.534) (width 0.75) (layer "B.Cu") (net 4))
 (segment (start 139.192001 67.056001) (end 131.572001 67.056001) (width 0.75) (layer "B.Cu") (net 4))
 (segment (start 131.572001 67.056001) (end 131.572 67.056) (width 0.75) (layer "B.Cu") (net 4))
 (segment (start 141 72.868) (end 143.002 70.866) (width 0.75) (layer "B.Cu") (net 4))
 (segment (start 131.572 67.056) (end 130.302 65.786) (width 0.75) (layer "B.Cu") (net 4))
 (segment (start 123.19 78.105) (end 123.19 80.264) (width 0.75) (layer "B.Cu") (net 4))
 (segment (start 109.073 66.147) (end 109.601 66.675) (width 0.75) (layer "B.Cu") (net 4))
 (segment (start 124.46 81.534) (end 135.466 81.534) (width 0.75) (layer "B.Cu") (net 4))
 (segment (start 143.002 70.866) (end 144.018 70.866) (width 0.75) (layer "B.Cu") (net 4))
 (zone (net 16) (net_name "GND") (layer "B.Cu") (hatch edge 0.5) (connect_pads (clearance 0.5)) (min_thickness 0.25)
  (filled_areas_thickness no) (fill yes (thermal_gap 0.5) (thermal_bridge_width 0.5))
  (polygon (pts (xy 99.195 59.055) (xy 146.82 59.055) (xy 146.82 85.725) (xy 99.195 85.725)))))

